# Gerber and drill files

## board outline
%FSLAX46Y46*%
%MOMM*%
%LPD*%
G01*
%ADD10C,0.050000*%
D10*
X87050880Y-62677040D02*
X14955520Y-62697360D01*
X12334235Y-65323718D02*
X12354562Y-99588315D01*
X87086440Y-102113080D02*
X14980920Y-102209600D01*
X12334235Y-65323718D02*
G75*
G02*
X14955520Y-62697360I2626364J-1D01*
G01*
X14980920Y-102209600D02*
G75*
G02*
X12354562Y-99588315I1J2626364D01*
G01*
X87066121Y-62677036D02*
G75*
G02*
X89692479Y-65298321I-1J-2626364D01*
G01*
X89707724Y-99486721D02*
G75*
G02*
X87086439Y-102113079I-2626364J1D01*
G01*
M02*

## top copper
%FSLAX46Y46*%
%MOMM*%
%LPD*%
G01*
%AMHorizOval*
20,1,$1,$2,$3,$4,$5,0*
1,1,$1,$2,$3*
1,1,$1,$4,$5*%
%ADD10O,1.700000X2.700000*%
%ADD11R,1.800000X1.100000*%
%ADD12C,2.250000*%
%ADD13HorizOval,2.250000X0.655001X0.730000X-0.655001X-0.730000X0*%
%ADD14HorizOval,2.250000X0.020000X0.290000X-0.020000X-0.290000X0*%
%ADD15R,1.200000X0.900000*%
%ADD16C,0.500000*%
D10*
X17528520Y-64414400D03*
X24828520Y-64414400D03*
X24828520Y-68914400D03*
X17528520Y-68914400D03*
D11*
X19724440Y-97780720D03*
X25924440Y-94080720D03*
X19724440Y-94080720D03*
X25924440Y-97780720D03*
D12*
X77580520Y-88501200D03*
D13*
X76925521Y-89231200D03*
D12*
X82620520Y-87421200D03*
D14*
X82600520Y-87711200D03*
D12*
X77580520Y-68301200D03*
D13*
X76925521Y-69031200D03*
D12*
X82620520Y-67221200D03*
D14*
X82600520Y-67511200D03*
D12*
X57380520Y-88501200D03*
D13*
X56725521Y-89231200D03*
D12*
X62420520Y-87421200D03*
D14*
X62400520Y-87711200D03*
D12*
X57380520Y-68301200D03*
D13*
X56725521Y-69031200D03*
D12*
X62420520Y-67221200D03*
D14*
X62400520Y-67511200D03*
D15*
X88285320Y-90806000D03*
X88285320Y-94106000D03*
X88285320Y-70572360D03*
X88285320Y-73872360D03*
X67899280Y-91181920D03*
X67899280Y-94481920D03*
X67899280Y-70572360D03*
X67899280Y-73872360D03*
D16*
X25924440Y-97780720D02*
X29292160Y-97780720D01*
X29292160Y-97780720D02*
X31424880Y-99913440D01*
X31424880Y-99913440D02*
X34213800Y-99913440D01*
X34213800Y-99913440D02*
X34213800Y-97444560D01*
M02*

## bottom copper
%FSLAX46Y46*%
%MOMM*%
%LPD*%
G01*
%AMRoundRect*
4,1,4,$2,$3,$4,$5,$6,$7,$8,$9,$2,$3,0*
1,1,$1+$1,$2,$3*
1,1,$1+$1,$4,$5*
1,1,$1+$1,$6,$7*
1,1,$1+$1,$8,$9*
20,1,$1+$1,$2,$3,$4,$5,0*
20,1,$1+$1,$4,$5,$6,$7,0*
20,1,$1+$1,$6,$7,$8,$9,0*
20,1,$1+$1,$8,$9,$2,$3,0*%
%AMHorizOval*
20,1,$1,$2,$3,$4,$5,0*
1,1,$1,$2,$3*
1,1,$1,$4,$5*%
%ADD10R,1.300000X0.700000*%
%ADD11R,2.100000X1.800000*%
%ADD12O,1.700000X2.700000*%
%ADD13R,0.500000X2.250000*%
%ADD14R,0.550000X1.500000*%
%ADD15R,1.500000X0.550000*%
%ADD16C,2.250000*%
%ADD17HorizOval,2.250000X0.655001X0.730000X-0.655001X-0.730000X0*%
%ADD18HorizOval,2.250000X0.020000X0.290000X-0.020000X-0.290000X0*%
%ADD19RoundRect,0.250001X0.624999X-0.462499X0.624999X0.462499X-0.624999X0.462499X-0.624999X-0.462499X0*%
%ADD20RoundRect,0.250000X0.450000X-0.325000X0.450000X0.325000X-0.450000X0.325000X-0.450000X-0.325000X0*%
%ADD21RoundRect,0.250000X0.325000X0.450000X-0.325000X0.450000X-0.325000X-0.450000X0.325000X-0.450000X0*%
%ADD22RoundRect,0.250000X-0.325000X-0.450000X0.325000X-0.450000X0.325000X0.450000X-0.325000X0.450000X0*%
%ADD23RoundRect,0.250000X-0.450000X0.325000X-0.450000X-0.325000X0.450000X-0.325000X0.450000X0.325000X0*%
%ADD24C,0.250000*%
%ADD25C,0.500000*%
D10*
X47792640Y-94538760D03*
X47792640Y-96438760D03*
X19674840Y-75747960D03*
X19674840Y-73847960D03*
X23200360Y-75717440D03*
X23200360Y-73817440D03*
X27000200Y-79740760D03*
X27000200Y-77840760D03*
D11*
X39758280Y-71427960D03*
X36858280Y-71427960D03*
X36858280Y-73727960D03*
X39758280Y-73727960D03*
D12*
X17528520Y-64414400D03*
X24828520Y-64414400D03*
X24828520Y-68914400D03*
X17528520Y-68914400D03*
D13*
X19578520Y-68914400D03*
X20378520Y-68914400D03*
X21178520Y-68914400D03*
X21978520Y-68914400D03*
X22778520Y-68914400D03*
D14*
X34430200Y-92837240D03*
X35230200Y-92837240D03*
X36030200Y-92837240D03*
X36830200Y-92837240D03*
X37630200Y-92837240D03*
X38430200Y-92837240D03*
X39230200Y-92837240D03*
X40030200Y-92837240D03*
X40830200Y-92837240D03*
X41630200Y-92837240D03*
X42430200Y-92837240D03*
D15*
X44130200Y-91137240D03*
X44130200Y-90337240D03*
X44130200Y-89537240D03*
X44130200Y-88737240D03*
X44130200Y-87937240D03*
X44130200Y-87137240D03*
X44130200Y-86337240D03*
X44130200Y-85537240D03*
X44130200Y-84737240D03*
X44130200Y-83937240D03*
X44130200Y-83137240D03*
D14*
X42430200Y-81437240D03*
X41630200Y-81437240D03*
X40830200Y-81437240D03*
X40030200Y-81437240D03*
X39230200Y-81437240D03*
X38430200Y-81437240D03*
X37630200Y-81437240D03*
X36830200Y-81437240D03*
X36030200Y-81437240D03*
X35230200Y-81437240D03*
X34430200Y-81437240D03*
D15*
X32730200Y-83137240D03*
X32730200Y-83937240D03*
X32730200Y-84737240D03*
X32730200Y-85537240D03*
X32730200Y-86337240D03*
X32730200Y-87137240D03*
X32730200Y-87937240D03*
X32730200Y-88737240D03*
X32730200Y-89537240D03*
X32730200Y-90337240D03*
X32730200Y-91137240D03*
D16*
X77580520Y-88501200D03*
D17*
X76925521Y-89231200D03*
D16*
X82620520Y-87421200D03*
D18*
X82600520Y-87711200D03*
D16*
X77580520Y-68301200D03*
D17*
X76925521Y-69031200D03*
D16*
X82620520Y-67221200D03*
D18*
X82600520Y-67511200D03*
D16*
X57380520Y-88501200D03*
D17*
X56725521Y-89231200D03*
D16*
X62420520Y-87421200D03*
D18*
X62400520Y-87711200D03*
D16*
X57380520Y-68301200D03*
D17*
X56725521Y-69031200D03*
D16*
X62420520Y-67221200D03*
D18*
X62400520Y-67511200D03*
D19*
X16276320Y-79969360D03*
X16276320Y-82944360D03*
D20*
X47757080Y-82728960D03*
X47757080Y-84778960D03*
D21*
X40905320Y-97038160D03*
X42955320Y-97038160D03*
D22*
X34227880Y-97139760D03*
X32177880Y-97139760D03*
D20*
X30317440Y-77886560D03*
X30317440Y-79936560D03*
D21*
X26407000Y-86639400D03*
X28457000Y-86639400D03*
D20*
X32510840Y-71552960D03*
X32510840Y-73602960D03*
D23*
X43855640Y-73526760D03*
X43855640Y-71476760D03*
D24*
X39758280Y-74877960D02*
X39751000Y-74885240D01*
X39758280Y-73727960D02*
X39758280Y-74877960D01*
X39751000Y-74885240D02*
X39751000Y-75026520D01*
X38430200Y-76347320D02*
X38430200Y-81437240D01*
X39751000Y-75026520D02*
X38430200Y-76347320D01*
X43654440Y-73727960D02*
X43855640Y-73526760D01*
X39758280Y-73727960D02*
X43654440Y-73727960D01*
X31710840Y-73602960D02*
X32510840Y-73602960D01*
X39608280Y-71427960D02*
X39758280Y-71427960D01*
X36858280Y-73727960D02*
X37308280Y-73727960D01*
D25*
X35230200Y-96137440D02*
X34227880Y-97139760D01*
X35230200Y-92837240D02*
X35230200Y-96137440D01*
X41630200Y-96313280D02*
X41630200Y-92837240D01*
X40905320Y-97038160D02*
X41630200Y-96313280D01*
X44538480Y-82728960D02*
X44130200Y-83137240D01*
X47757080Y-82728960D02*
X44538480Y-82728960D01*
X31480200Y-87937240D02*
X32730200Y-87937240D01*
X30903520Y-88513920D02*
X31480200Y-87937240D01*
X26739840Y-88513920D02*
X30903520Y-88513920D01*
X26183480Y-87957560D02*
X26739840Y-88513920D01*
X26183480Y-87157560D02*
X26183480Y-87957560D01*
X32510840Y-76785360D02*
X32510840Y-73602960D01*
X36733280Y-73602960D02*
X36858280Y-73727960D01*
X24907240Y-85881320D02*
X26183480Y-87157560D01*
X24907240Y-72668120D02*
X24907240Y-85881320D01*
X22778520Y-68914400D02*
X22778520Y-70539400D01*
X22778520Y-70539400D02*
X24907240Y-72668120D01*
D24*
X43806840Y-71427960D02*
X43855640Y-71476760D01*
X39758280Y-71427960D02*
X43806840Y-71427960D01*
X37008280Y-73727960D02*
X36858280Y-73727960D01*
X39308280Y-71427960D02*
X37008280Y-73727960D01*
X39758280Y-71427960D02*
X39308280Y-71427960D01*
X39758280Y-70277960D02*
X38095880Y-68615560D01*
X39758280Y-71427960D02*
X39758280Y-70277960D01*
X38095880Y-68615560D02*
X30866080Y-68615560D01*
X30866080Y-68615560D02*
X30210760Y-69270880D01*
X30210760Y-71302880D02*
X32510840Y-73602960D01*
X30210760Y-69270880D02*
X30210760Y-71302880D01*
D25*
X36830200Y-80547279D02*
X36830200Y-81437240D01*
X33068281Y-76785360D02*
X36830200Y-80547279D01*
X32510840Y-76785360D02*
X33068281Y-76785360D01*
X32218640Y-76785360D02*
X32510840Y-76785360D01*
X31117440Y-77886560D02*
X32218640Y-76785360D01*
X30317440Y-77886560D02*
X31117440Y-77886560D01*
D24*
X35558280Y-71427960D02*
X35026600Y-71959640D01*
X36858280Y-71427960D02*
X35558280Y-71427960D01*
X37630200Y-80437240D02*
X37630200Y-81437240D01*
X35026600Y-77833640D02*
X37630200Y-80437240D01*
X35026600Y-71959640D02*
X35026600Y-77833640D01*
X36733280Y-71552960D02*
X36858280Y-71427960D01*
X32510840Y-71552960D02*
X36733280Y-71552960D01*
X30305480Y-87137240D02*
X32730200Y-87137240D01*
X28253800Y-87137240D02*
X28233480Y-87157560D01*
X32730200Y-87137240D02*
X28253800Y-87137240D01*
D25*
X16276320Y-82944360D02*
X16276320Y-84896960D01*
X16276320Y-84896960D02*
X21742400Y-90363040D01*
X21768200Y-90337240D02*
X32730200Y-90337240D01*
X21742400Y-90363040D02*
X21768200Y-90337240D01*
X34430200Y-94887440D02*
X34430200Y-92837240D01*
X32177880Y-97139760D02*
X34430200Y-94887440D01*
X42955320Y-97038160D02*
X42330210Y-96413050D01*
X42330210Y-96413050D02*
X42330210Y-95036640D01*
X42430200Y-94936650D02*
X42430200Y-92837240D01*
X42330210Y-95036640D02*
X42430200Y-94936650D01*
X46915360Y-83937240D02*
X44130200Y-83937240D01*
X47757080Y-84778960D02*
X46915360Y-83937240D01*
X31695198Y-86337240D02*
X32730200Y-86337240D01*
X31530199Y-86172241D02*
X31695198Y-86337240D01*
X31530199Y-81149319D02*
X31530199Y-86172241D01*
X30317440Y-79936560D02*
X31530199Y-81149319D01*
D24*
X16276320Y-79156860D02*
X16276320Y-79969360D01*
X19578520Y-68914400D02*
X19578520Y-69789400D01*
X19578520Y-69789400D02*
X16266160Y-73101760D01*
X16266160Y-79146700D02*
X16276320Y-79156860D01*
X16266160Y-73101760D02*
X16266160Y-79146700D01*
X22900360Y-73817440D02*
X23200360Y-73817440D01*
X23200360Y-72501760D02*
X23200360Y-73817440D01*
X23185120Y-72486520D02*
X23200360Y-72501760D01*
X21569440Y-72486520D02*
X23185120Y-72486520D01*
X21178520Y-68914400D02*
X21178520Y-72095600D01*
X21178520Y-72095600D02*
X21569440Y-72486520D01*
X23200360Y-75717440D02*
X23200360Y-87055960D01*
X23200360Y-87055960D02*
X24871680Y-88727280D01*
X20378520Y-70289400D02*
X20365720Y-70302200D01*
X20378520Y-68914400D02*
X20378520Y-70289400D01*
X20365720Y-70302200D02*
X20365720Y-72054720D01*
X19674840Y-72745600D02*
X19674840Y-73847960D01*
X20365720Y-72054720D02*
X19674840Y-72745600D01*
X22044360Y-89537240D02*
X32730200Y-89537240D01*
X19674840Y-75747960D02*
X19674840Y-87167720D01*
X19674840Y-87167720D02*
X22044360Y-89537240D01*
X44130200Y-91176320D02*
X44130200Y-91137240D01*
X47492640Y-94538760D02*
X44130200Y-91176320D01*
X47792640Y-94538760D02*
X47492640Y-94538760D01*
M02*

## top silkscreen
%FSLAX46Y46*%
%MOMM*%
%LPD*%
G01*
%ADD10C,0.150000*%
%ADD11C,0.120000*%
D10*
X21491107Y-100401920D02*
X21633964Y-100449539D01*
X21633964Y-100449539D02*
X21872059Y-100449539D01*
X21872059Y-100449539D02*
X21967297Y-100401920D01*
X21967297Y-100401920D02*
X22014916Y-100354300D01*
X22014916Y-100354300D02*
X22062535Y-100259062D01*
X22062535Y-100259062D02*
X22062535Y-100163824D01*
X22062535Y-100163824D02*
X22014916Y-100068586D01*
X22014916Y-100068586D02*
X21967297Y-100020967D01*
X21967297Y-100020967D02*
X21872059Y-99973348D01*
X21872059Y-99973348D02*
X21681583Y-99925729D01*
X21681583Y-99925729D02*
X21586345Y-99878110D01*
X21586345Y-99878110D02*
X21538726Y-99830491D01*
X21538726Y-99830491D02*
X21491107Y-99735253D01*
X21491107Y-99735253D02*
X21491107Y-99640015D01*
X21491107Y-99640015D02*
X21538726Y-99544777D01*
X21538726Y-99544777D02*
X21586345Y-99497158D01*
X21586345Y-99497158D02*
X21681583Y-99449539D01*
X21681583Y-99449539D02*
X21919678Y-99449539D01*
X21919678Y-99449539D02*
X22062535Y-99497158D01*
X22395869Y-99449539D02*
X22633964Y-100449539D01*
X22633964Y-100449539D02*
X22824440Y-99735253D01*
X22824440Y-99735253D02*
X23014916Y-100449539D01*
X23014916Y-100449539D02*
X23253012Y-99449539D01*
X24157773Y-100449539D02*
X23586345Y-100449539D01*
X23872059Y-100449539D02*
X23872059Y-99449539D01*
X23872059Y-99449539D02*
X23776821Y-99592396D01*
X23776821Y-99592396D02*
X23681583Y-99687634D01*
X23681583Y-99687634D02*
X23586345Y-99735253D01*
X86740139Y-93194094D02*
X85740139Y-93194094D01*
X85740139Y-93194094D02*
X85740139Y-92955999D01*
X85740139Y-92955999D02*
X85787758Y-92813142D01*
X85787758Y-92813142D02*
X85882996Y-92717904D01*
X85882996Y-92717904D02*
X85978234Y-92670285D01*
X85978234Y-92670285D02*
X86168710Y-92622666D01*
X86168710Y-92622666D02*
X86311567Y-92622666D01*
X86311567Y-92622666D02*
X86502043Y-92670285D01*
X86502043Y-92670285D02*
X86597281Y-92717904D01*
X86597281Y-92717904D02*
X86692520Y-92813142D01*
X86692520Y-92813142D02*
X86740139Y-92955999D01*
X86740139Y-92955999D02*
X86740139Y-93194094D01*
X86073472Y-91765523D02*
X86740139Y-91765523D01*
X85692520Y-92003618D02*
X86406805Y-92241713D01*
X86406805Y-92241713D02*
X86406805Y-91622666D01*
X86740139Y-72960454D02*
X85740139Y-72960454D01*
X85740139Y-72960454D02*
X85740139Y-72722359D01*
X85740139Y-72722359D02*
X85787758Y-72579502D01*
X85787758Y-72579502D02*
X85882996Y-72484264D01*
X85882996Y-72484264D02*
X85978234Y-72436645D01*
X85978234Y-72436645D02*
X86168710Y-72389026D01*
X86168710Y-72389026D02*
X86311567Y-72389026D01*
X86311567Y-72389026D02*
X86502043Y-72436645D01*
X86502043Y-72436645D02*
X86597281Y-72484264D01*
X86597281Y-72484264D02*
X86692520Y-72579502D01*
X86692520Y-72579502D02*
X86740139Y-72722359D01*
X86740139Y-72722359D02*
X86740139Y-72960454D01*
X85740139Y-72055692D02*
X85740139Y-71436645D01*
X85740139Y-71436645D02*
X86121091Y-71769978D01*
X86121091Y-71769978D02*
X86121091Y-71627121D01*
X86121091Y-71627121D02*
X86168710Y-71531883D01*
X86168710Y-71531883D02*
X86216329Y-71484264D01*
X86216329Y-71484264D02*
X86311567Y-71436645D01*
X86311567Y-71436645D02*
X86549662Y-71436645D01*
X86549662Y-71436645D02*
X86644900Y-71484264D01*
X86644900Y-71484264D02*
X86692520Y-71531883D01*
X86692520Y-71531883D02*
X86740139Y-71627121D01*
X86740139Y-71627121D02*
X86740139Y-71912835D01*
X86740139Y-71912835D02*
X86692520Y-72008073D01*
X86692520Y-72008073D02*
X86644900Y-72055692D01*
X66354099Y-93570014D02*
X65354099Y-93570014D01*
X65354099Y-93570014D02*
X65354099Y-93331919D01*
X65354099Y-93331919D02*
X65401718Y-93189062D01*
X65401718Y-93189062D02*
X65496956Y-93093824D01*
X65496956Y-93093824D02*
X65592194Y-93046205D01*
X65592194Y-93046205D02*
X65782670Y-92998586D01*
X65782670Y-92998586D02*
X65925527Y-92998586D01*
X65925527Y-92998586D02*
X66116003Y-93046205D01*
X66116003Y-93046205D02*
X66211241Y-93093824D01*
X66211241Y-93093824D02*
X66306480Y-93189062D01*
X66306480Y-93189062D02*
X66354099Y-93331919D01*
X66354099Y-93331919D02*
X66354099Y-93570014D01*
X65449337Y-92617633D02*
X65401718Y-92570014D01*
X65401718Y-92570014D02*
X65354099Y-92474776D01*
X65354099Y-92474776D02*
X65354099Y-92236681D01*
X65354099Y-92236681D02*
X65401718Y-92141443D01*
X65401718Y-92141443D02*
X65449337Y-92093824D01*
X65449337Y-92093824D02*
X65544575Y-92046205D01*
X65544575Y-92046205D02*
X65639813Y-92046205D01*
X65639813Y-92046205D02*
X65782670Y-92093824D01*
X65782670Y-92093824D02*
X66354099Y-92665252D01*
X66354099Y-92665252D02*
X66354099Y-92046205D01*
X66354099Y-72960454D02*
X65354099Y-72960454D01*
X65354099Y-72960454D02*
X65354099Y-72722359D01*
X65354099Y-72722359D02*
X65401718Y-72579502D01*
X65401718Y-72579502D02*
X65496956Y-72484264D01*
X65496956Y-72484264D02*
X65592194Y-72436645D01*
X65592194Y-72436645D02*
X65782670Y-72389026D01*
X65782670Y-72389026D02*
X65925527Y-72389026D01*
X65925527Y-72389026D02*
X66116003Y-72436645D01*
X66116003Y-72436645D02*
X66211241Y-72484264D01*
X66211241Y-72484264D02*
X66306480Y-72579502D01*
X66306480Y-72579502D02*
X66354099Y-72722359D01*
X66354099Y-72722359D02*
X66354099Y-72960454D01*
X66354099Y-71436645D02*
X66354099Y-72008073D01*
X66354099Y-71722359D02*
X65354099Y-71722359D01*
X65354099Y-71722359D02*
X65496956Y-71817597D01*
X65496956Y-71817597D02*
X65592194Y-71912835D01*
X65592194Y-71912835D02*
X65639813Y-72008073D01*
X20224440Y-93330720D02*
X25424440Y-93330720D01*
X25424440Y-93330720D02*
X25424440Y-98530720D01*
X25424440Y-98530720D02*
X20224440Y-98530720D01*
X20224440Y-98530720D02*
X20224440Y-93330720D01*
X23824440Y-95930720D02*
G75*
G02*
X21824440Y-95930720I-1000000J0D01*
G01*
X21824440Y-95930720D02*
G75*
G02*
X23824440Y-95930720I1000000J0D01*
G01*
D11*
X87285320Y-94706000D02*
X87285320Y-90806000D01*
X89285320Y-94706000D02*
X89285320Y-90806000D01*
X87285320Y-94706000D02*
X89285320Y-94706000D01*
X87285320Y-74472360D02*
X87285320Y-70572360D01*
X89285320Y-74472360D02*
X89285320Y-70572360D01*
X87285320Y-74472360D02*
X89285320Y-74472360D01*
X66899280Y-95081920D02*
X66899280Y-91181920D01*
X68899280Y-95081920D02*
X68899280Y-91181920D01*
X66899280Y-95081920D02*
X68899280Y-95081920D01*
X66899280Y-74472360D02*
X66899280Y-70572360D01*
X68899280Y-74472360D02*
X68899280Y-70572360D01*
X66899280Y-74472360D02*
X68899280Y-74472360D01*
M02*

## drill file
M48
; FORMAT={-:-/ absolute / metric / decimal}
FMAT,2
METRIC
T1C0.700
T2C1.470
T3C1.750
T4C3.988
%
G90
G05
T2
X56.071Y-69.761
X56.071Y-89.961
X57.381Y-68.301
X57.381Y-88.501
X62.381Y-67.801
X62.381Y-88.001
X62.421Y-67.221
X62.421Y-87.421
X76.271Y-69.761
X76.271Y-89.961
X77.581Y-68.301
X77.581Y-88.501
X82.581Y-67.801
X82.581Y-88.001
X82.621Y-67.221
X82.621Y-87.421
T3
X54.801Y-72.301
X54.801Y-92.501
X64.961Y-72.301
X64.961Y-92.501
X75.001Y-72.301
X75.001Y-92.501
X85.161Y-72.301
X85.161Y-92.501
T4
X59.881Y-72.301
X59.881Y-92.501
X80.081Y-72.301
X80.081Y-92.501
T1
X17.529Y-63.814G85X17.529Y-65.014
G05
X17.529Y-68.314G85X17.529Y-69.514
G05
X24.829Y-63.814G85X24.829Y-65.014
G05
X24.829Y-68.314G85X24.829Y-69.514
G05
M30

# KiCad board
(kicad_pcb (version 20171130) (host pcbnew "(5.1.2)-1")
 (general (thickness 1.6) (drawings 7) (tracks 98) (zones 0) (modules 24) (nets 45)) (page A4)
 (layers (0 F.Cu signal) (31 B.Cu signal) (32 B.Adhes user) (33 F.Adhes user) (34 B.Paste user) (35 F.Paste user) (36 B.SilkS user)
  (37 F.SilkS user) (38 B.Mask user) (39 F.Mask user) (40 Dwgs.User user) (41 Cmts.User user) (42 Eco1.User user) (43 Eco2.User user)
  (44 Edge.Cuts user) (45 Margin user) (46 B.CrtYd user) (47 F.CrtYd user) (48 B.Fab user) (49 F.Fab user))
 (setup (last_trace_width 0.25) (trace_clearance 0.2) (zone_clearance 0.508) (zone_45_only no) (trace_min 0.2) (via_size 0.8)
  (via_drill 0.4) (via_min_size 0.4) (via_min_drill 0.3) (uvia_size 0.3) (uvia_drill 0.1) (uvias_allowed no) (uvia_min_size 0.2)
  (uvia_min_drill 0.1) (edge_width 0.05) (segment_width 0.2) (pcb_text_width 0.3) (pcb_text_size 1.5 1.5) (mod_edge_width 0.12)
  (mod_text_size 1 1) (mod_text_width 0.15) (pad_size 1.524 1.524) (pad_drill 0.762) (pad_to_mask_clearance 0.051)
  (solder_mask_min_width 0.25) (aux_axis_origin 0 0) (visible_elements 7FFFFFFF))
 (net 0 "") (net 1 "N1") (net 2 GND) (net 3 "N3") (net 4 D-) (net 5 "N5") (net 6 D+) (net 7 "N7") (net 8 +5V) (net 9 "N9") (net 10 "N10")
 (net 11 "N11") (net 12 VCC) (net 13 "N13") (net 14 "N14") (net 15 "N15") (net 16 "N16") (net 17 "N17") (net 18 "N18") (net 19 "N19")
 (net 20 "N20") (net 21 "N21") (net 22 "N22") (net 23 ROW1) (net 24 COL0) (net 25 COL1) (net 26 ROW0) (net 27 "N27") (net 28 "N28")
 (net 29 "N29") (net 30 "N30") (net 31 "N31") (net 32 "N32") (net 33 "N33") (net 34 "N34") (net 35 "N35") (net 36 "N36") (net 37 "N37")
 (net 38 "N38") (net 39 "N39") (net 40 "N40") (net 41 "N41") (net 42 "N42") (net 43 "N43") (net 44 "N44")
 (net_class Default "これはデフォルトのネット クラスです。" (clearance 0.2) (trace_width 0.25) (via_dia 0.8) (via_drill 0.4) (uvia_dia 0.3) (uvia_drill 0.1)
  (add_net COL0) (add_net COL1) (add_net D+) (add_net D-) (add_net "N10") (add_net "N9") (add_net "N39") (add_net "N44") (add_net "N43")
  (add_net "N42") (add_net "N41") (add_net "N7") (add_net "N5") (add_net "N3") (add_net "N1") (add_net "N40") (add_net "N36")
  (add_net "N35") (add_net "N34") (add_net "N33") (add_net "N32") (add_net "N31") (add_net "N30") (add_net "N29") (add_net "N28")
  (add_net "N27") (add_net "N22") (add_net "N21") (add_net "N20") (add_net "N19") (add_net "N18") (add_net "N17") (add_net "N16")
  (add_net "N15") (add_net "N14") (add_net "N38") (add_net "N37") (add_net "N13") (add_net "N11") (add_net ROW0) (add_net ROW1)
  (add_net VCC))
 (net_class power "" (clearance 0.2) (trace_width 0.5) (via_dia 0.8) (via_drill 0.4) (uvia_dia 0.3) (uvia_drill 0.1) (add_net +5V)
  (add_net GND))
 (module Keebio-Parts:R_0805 (layer B.Cu) (at 47.79264 95.48876 90)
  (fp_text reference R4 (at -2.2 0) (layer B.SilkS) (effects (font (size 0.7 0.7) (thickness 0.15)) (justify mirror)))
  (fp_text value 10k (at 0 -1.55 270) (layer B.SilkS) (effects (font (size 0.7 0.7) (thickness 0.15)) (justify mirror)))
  (pad 2 smd rect (at 0.95 0 90) (size 0.7 1.3) (layers B.Cu B.Paste B.Mask) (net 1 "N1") (clearance 0.1))
  (pad 1 smd rect (at -0.95 0 90) (size 0.7 1.3) (layers B.Cu B.Paste B.Mask) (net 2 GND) (clearance 0.1)))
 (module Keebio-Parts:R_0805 (layer B.Cu) (at 19.67484 74.79796 90)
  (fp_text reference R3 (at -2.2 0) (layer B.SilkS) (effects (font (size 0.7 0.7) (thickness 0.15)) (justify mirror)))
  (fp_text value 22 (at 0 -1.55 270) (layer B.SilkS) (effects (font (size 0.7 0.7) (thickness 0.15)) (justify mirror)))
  (pad 1 smd rect (at -0.95 0 90) (size 0.7 1.3) (layers B.Cu B.Paste B.Mask) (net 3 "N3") (clearance 0.1))
  (pad 2 smd rect (at 0.95 0 90) (size 0.7 1.3) (layers B.Cu B.Paste B.Mask) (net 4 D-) (clearance 0.1)))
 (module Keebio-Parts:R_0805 (layer B.Cu) (at 23.20036 74.76744 90)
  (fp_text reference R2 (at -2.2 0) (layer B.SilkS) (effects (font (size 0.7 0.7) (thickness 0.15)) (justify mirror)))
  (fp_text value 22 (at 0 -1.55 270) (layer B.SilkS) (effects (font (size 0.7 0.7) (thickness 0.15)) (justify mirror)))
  (pad 1 smd rect (at -0.95 0 90) (size 0.7 1.3) (layers B.Cu B.Paste B.Mask) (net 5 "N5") (clearance 0.1))
  (pad 2 smd rect (at 0.95 0 90) (size 0.7 1.3) (layers B.Cu B.Paste B.Mask) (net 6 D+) (clearance 0.1)))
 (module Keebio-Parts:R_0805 (layer B.Cu) (at 27.0002 78.79076 90)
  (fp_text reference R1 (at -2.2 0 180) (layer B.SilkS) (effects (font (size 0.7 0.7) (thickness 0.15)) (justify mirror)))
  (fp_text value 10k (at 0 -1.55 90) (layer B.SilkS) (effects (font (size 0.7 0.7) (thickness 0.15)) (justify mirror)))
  (pad 1 smd rect (at -0.95 0 90) (size 0.7 1.3) (layers B.Cu B.Paste B.Mask) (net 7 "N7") (clearance 0.1))
  (pad 2 smd rect (at 0.95 0 90) (size 0.7 1.3) (layers B.Cu B.Paste B.Mask) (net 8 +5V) (clearance 0.1)))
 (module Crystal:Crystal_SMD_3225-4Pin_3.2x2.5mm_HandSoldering (layer B.Cu) (at 38.30828 72.57796 180)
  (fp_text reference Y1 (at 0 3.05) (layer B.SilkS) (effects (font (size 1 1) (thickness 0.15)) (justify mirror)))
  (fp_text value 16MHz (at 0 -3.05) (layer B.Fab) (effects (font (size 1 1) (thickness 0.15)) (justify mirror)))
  (pad 4 smd rect (at -1.45 1.15 180) (size 2.1 1.8) (layers B.Cu B.Paste B.Mask) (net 2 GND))
  (pad 3 smd rect (at 1.45 1.15 180) (size 2.1 1.8) (layers B.Cu B.Paste B.Mask) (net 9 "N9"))
  (pad 2 smd rect (at 1.45 -1.15 180) (size 2.1 1.8) (layers B.Cu B.Paste B.Mask) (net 2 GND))
  (pad 1 smd rect (at -1.45 -1.15 180) (size 2.1 1.8) (layers B.Cu B.Paste B.Mask) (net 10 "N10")))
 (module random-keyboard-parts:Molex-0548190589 (layer B.Cu) (at 21.17852 64.4144 270)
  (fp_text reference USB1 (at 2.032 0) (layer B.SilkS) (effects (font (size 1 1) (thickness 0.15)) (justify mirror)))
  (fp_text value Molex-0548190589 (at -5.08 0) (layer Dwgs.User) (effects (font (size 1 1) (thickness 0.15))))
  (pad 6 thru_hole oval (at 0 3.65 270) (size 2.7 1.7) (drill oval 1.9 0.7) (layers *.Cu *.Mask) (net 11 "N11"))
  (pad 6 thru_hole oval (at 0 -3.65 270) (size 2.7 1.7) (drill oval 1.9 0.7) (layers *.Cu *.Mask) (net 11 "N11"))
  (pad 6 thru_hole oval (at 4.5 -3.65 270) (size 2.7 1.7) (drill oval 1.9 0.7) (layers *.Cu *.Mask) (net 11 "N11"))
  (pad 6 thru_hole oval (at 4.5 3.65 270) (size 2.7 1.7) (drill oval 1.9 0.7) (layers *.Cu *.Mask) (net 11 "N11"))
  (pad 5 smd rect (at 4.5 1.6 270) (size 2.25 0.5) (layers B.Cu B.Paste B.Mask) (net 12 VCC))
  (pad 4 smd rect (at 4.5 0.8 270) (size 2.25 0.5) (layers B.Cu B.Paste B.Mask) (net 4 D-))
  (pad 3 smd rect (at 4.5 0 270) (size 2.25 0.5) (layers B.Cu B.Paste B.Mask) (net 6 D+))
  (pad 2 smd rect (at 4.5 -0.8 270) (size 2.25 0.5) (layers B.Cu B.Paste B.Mask) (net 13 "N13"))
  (pad 1 smd rect (at 4.5 -1.6 270) (size 2.25 0.5) (layers B.Cu B.Paste B.Mask) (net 2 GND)))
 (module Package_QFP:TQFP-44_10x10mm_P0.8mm (layer B.Cu) (at 38.4302 87.13724)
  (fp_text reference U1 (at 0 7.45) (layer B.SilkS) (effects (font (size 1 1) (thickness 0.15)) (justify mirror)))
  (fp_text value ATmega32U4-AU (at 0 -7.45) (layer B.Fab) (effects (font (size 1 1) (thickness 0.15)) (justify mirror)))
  (pad 44 smd rect (at -4 5.7 270) (size 1.5 0.55) (layers B.Cu B.Paste B.Mask) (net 8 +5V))
  (pad 43 smd rect (at -3.2 5.7 270) (size 1.5 0.55) (layers B.Cu B.Paste B.Mask) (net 2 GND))
  (pad 42 smd rect (at -2.4 5.7 270) (size 1.5 0.55) (layers B.Cu B.Paste B.Mask) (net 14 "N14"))
  (pad 41 smd rect (at -1.6 5.7 270) (size 1.5 0.55) (layers B.Cu B.Paste B.Mask) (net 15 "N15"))
  (pad 40 smd rect (at -0.8 5.7 270) (size 1.5 0.55) (layers B.Cu B.Paste B.Mask) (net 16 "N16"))
  (pad 39 smd rect (at 0 5.7 270) (size 1.5 0.55) (layers B.Cu B.Paste B.Mask) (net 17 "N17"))
  (pad 38 smd rect (at 0.8 5.7 270) (size 1.5 0.55) (layers B.Cu B.Paste B.Mask) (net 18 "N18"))
  (pad 37 smd rect (at 1.6 5.7 270) (size 1.5 0.55) (layers B.Cu B.Paste B.Mask) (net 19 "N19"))
  (pad 36 smd rect (at 2.4 5.7 270) (size 1.5 0.55) (layers B.Cu B.Paste B.Mask) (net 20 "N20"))
  (pad 35 smd rect (at 3.2 5.7 270) (size 1.5 0.55) (layers B.Cu B.Paste B.Mask) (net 2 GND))
  (pad 34 smd rect (at 4 5.7 270) (size 1.5 0.55) (layers B.Cu B.Paste B.Mask) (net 8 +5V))
  (pad 33 smd rect (at 5.7 4) (size 1.5 0.55) (layers B.Cu B.Paste B.Mask) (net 1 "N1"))
  (pad 32 smd rect (at 5.7 3.2) (size 1.5 0.55) (layers B.Cu B.Paste B.Mask) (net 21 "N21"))
  (pad 31 smd rect (at 5.7 2.4) (size 1.5 0.55) (layers B.Cu B.Paste B.Mask) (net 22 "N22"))
  (pad 30 smd rect (at 5.7 1.6) (size 1.5 0.55) (layers B.Cu B.Paste B.Mask) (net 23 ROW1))
  (pad 29 smd rect (at 5.7 0.8) (size 1.5 0.55) (layers B.Cu B.Paste B.Mask) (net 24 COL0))
  (pad 28 smd rect (at 5.7 0) (size 1.5 0.55) (layers B.Cu B.Paste B.Mask) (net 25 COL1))
  (pad 27 smd rect (at 5.7 -0.8) (size 1.5 0.55) (layers B.Cu B.Paste B.Mask) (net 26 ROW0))
  (pad 26 smd rect (at 5.7 -1.6) (size 1.5 0.55) (layers B.Cu B.Paste B.Mask) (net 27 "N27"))
  (pad 25 smd rect (at 5.7 -2.4) (size 1.5 0.55) (layers B.Cu B.Paste B.Mask) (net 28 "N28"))
  (pad 24 smd rect (at 5.7 -3.2) (size 1.5 0.55) (layers B.Cu B.Paste B.Mask) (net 8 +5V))
  (pad 23 smd rect (at 5.7 -4) (size 1.5 0.55) (layers B.Cu B.Paste B.Mask) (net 2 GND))
  (pad 22 smd rect (at 4 -5.7 270) (size 1.5 0.55) (layers B.Cu B.Paste B.Mask) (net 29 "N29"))
  (pad 21 smd rect (at 3.2 -5.7 270) (size 1.5 0.55) (layers B.Cu B.Paste B.Mask) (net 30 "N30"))
  (pad 20 smd rect (at 2.4 -5.7 270) (size 1.5 0.55) (layers B.Cu B.Paste B.Mask) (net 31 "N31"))
  (pad 19 smd rect (at 1.6 -5.7 270) (size 1.5 0.55) (layers B.Cu B.Paste B.Mask) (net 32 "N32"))
  (pad 18 smd rect (at 0.8 -5.7 270) (size 1.5 0.55) (layers B.Cu B.Paste B.Mask) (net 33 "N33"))
  (pad 17 smd rect (at 0 -5.7 270) (size 1.5 0.55) (layers B.Cu B.Paste B.Mask) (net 10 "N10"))
  (pad 16 smd rect (at -0.8 -5.7 270) (size 1.5 0.55) (layers B.Cu B.Paste B.Mask) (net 9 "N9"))
  (pad 15 smd rect (at -1.6 -5.7 270) (size 1.5 0.55) (layers B.Cu B.Paste B.Mask) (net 2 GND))
  (pad 14 smd rect (at -2.4 -5.7 270) (size 1.5 0.55) (layers B.Cu B.Paste B.Mask) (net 8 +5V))
  (pad 13 smd rect (at -3.2 -5.7 270) (size 1.5 0.55) (layers B.Cu B.Paste B.Mask) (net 7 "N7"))
  (pad 12 smd rect (at -4 -5.7 270) (size 1.5 0.55) (layers B.Cu B.Paste B.Mask) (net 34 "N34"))
  (pad 11 smd rect (at -5.7 -4) (size 1.5 0.55) (layers B.Cu B.Paste B.Mask) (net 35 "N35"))
  (pad 10 smd rect (at -5.7 -3.2) (size 1.5 0.55) (layers B.Cu B.Paste B.Mask) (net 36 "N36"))
  (pad 9 smd rect (at -5.7 -2.4) (size 1.5 0.55) (layers B.Cu B.Paste B.Mask) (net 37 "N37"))
  (pad 8 smd rect (at -5.7 -1.6) (size 1.5 0.55) (layers B.Cu B.Paste B.Mask) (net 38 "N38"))
  (pad 7 smd rect (at -5.7 -0.8) (size 1.5 0.55) (layers B.Cu B.Paste B.Mask) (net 8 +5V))
  (pad 6 smd rect (at -5.7 0) (size 1.5 0.55) (layers B.Cu B.Paste B.Mask) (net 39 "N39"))
  (pad 5 smd rect (at -5.7 0.8) (size 1.5 0.55) (layers B.Cu B.Paste B.Mask) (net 2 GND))
  (pad 4 smd rect (at -5.7 1.6) (size 1.5 0.55) (layers B.Cu B.Paste B.Mask) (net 5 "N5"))
  (pad 3 smd rect (at -5.7 2.4) (size 1.5 0.55) (layers B.Cu B.Paste B.Mask) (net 3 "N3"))
  (pad 2 smd rect (at -5.7 3.2) (size 1.5 0.55) (layers B.Cu B.Paste B.Mask) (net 8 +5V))
  (pad 1 smd rect (at -5.7 4) (size 1.5 0.55) (layers B.Cu B.Paste B.Mask) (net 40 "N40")))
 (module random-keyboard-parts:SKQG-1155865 (layer F.Cu) (at 22.82444 95.93072)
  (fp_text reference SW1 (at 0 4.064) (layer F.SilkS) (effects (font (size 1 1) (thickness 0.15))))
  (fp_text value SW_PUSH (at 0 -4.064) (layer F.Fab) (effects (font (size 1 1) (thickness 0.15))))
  (fp_line (start -2.6 -2.6) (end 2.6 -2.6) (layer F.SilkS) (width 0.15))
  (fp_line (start 2.6 -2.6) (end 2.6 2.6) (layer F.SilkS) (width 0.15))
  (fp_line (start 2.6 2.6) (end -2.6 2.6) (layer F.SilkS) (width 0.15))
  (fp_line (start -2.6 2.6) (end -2.6 -2.6) (layer F.SilkS) (width 0.15))
  (fp_circle (center 0 0) (end 1 0) (layer F.SilkS) (width 0.15))
  (pad 4 smd rect (at -3.1 1.85) (size 1.8 1.1) (layers F.Cu F.Paste F.Mask))
  (pad 3 smd rect (at 3.1 -1.85) (size 1.8 1.1) (layers F.Cu F.Paste F.Mask))
  (pad 2 smd rect (at -3.1 -1.85) (size 1.8 1.1) (layers F.Cu F.Paste F.Mask) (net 7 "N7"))
  (pad 1 smd rect (at 3.1 1.85) (size 1.8 1.1) (layers F.Cu F.Paste F.Mask) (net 2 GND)))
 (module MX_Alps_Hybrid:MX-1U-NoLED (layer F.Cu) (at 80.08052 92.5012)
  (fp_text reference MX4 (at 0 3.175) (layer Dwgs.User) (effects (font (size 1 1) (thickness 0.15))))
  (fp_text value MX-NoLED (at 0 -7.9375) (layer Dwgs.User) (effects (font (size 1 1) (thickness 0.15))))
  (pad "" np_thru_hole circle (at 5.08 0 48.0996) (size 1.75 1.75) (drill 1.75) (layers *.Cu *.Mask))
  (pad "" np_thru_hole circle (at -5.08 0 48.0996) (size 1.75 1.75) (drill 1.75) (layers *.Cu *.Mask))
  (pad 1 thru_hole circle (at -2.5 -4) (size 2.25 2.25) (drill 1.47) (layers *.Cu B.Mask) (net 25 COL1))
  (pad "" np_thru_hole circle (at 0 0) (size 3.9878 3.9878) (drill 3.9878) (layers *.Cu *.Mask))
  (pad 1 thru_hole oval (at -3.81 -2.54 48.0996) (size 4.211556 2.25) (drill 1.47 (offset 0.980778 0)) (layers *.Cu B.Mask) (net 25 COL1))
  (pad 2 thru_hole circle (at 2.54 -5.08) (size 2.25 2.25) (drill 1.47) (layers *.Cu B.Mask) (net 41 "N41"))
  (pad 2 thru_hole oval (at 2.5 -4.5 86.0548) (size 2.831378 2.25) (drill 1.47 (offset 0.290689 0)) (layers *.Cu B.Mask) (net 41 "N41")))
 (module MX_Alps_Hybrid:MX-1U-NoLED (layer F.Cu) (at 80.08052 72.3012)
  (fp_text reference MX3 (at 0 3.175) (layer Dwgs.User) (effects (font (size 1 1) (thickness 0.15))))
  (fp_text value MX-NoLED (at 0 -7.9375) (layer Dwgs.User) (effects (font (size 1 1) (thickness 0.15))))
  (pad "" np_thru_hole circle (at 5.08 0 48.0996) (size 1.75 1.75) (drill 1.75) (layers *.Cu *.Mask))
  (pad "" np_thru_hole circle (at -5.08 0 48.0996) (size 1.75 1.75) (drill 1.75) (layers *.Cu *.Mask))
  (pad 1 thru_hole circle (at -2.5 -4) (size 2.25 2.25) (drill 1.47) (layers *.Cu B.Mask) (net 24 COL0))
  (pad "" np_thru_hole circle (at 0 0) (size 3.9878 3.9878) (drill 3.9878) (layers *.Cu *.Mask))
  (pad 1 thru_hole oval (at -3.81 -2.54 48.0996) (size 4.211556 2.25) (drill 1.47 (offset 0.980778 0)) (layers *.Cu B.Mask) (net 24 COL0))
  (pad 2 thru_hole circle (at 2.54 -5.08) (size 2.25 2.25) (drill 1.47) (layers *.Cu B.Mask) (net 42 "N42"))
  (pad 2 thru_hole oval (at 2.5 -4.5 86.0548) (size 2.831378 2.25) (drill 1.47 (offset 0.290689 0)) (layers *.Cu B.Mask) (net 42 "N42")))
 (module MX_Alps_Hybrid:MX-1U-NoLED (layer F.Cu) (at 59.88052 92.5012)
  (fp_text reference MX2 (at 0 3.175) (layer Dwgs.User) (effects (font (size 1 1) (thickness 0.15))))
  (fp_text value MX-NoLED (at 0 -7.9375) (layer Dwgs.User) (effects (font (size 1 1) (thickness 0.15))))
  (pad "" np_thru_hole circle (at 5.08 0 48.0996) (size 1.75 1.75) (drill 1.75) (layers *.Cu *.Mask))
  (pad "" np_thru_hole circle (at -5.08 0 48.0996) (size 1.75 1.75) (drill 1.75) (layers *.Cu *.Mask))
  (pad 1 thru_hole circle (at -2.5 -4) (size 2.25 2.25) (drill 1.47) (layers *.Cu B.Mask) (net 25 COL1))
  (pad "" np_thru_hole circle (at 0 0) (size 3.9878 3.9878) (drill 3.9878) (layers *.Cu *.Mask))
  (pad 1 thru_hole oval (at -3.81 -2.54 48.0996) (size 4.211556 2.25) (drill 1.47 (offset 0.980778 0)) (layers *.Cu B.Mask) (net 25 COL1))
  (pad 2 thru_hole circle (at 2.54 -5.08) (size 2.25 2.25) (drill 1.47) (layers *.Cu B.Mask) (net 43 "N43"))
  (pad 2 thru_hole oval (at 2.5 -4.5 86.0548) (size 2.831378 2.25) (drill 1.47 (offset 0.290689 0)) (layers *.Cu B.Mask) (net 43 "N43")))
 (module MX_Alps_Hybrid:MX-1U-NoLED (layer F.Cu) (at 59.88052 72.3012)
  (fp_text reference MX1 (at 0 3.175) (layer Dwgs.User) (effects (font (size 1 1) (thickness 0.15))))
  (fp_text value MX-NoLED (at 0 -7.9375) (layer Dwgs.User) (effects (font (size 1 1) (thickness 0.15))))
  (pad "" np_thru_hole circle (at 5.08 0 48.0996) (size 1.75 1.75) (drill 1.75) (layers *.Cu *.Mask))
  (pad "" np_thru_hole circle (at -5.08 0 48.0996) (size 1.75 1.75) (drill 1.75) (layers *.Cu *.Mask))
  (pad 1 thru_hole circle (at -2.5 -4) (size 2.25 2.25) (drill 1.47) (layers *.Cu B.Mask) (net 24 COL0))
  (pad "" np_thru_hole circle (at 0 0) (size 3.9878 3.9878) (drill 3.9878) (layers *.Cu *.Mask))
  (pad 1 thru_hole oval (at -3.81 -2.54 48.0996) (size 4.211556 2.25) (drill 1.47 (offset 0.980778 0)) (layers *.Cu B.Mask) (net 24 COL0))
  (pad 2 thru_hole circle (at 2.54 -5.08) (size 2.25 2.25) (drill 1.47) (layers *.Cu B.Mask) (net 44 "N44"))
  (pad 2 thru_hole oval (at 2.5 -4.5 86.0548) (size 2.831378 2.25) (drill 1.47 (offset 0.290689 0)) (layers *.Cu B.Mask) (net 44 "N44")))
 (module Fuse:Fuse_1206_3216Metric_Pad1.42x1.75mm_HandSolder (layer B.Cu) (at 16.27632 81.45686 90)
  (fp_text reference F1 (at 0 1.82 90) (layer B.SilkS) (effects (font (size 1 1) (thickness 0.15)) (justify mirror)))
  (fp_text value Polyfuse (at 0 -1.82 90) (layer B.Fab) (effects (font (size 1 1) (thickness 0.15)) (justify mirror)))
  (pad 2 smd roundrect (at 1.4875 0 90) (size 1.425 1.75) (layers B.Cu B.Paste B.Mask) (roundrect_rratio 0.175439) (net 12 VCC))
  (pad 1 smd roundrect (at -1.4875 0 90) (size 1.425 1.75) (layers B.Cu B.Paste B.Mask) (roundrect_rratio 0.175439) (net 8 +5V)))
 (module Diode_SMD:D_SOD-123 (layer F.Cu) (at 88.28532 92.456 90)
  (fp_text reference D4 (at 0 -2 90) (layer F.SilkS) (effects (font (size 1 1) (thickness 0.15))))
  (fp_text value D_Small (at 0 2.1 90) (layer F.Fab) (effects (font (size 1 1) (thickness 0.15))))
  (fp_line (start -2.25 -1) (end 1.65 -1) (layer F.SilkS) (width 0.12))
  (fp_line (start -2.25 1) (end 1.65 1) (layer F.SilkS) (width 0.12))
  (fp_line (start -2.25 -1) (end -2.25 1) (layer F.SilkS) (width 0.12))
  (pad 2 smd rect (at 1.65 0 90) (size 0.9 1.2) (layers F.Cu F.Paste F.Mask) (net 41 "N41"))
  (pad 1 smd rect (at -1.65 0 90) (size 0.9 1.2) (layers F.Cu F.Paste F.Mask) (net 23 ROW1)))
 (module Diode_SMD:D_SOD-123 (layer F.Cu) (at 88.28532 72.22236 90)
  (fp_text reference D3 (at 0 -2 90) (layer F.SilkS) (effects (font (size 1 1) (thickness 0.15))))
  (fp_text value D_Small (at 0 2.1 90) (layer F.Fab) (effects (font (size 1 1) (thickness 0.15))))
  (fp_line (start -2.25 -1) (end 1.65 -1) (layer F.SilkS) (width 0.12))
  (fp_line (start -2.25 1) (end 1.65 1) (layer F.SilkS) (width 0.12))
  (fp_line (start -2.25 -1) (end -2.25 1) (layer F.SilkS) (width 0.12))
  (pad 2 smd rect (at 1.65 0 90) (size 0.9 1.2) (layers F.Cu F.Paste F.Mask) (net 42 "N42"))
  (pad 1 smd rect (at -1.65 0 90) (size 0.9 1.2) (layers F.Cu F.Paste F.Mask) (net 23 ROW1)))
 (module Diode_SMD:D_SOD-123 (layer F.Cu) (at 67.89928 92.83192 90)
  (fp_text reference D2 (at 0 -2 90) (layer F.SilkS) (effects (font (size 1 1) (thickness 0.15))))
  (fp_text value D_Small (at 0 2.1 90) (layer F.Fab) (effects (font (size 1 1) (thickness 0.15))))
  (fp_line (start -2.25 -1) (end 1.65 -1) (layer F.SilkS) (width 0.12))
  (fp_line (start -2.25 1) (end 1.65 1) (layer F.SilkS) (width 0.12))
  (fp_line (start -2.25 -1) (end -2.25 1) (layer F.SilkS) (width 0.12))
  (pad 2 smd rect (at 1.65 0 90) (size 0.9 1.2) (layers F.Cu F.Paste F.Mask) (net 43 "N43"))
  (pad 1 smd rect (at -1.65 0 90) (size 0.9 1.2) (layers F.Cu F.Paste F.Mask) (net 26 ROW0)))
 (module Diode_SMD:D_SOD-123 (layer F.Cu) (at 67.89928 72.22236 90)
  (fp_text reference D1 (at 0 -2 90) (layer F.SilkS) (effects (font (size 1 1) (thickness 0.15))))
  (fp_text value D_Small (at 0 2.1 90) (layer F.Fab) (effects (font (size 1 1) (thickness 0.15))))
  (fp_line (start -2.25 -1) (end 1.65 -1) (layer F.SilkS) (width 0.12))
  (fp_line (start -2.25 1) (end 1.65 1) (layer F.SilkS) (width 0.12))
  (fp_line (start -2.25 -1) (end -2.25 1) (layer F.SilkS) (width 0.12))
  (pad 2 smd rect (at 1.65 0 90) (size 0.9 1.2) (layers F.Cu F.Paste F.Mask) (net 44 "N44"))
  (pad 1 smd rect (at -1.65 0 90) (size 0.9 1.2) (layers F.Cu F.Paste F.Mask) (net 26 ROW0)))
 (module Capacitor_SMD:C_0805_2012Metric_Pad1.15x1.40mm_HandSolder (layer B.Cu) (at 47.75708 83.75396 90)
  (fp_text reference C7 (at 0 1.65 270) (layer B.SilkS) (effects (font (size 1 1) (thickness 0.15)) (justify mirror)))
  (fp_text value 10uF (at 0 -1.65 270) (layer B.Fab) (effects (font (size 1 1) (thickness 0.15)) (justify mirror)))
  (pad 2 smd roundrect (at 1.025 0 90) (size 1.15 1.4) (layers B.Cu B.Paste B.Mask) (roundrect_rratio 0.217391) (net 2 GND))
  (pad 1 smd roundrect (at -1.025 0 90) (size 1.15 1.4) (layers B.Cu B.Paste B.Mask) (roundrect_rratio 0.217391) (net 8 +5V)))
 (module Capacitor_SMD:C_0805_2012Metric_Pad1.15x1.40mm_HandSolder (layer B.Cu) (at 41.93032 97.03816 180)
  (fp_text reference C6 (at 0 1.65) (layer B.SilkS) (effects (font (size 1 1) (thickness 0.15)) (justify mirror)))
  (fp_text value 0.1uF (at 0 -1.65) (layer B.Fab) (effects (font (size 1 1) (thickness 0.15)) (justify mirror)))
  (pad 2 smd roundrect (at 1.025 0 180) (size 1.15 1.4) (layers B.Cu B.Paste B.Mask) (roundrect_rratio 0.217391) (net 2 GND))
  (pad 1 smd roundrect (at -1.025 0 180) (size 1.15 1.4) (layers B.Cu B.Paste B.Mask) (roundrect_rratio 0.217391) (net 8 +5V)))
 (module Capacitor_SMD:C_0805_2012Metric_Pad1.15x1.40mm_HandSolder (layer B.Cu) (at 33.20288 97.13976)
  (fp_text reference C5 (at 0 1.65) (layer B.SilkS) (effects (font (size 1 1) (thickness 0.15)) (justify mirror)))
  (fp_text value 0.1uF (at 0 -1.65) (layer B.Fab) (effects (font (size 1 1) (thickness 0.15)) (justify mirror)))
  (pad 2 smd roundrect (at 1.025 0) (size 1.15 1.4) (layers B.Cu B.Paste B.Mask) (roundrect_rratio 0.217391) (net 2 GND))
  (pad 1 smd roundrect (at -1.025 0) (size 1.15 1.4) (layers B.Cu B.Paste B.Mask) (roundrect_rratio 0.217391) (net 8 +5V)))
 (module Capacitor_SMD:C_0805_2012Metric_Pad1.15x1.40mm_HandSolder (layer B.Cu) (at 30.31744 78.91156 90)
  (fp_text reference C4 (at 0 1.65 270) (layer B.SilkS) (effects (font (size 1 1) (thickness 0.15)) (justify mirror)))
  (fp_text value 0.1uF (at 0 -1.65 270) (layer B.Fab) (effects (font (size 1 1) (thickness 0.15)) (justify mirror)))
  (pad 2 smd roundrect (at 1.025 0 90) (size 1.15 1.4) (layers B.Cu B.Paste B.Mask) (roundrect_rratio 0.217391) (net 2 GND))
  (pad 1 smd roundrect (at -1.025 0 90) (size 1.15 1.4) (layers B.Cu B.Paste B.Mask) (roundrect_rratio 0.217391) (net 8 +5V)))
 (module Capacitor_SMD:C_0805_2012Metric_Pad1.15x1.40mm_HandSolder (layer B.Cu) (at 27.432 86.6394 180)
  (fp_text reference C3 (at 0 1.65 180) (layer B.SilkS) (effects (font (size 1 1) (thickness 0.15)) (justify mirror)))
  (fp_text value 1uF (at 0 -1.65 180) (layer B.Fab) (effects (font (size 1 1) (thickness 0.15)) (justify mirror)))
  (pad 2 smd roundrect (at 1.025 0 180) (size 1.15 1.4) (layers B.Cu B.Paste B.Mask) (roundrect_rratio 0.217391) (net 2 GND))
  (pad 1 smd roundrect (at -1.025 0 180) (size 1.15 1.4) (layers B.Cu B.Paste B.Mask) (roundrect_rratio 0.217391) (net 39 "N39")))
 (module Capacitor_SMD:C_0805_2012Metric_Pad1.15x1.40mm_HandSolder (layer B.Cu) (at 32.51084 72.57796 90)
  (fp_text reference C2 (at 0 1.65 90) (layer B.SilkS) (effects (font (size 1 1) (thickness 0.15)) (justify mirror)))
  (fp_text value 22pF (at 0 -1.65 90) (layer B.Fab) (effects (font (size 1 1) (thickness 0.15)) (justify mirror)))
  (pad 2 smd roundrect (at 1.025 0 90) (size 1.15 1.4) (layers B.Cu B.Paste B.Mask) (roundrect_rratio 0.217391) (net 9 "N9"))
  (pad 1 smd roundrect (at -1.025 0 90) (size 1.15 1.4) (layers B.Cu B.Paste B.Mask) (roundrect_rratio 0.217391) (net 2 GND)))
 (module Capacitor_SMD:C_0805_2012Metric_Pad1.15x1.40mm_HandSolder (layer B.Cu) (at 43.85564 72.50176 270)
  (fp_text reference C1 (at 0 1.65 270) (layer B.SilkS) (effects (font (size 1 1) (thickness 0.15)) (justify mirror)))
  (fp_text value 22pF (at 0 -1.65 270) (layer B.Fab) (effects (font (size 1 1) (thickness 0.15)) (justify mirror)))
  (pad 2 smd roundrect (at 1.025 0 270) (size 1.15 1.4) (layers B.Cu B.Paste B.Mask) (roundrect_rratio 0.217391) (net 10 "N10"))
  (pad 1 smd roundrect (at -1.025 0 270) (size 1.15 1.4) (layers B.Cu B.Paste B.Mask) (roundrect_rratio 0.217391) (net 2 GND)))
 (gr_line (start 87.05088 62.67704) (end 14.95552 62.69736) (layer Edge.Cuts) (width 0.05))
 (gr_line (start 12.334235 65.323718) (end 12.354562 99.588315) (layer Edge.Cuts) (width 0.05))
 (gr_line (start 87.08644 102.11308) (end 14.98092 102.2096) (layer Edge.Cuts) (width 0.05))
 (gr_arc (start 14.960599 65.323719) (end 14.95552 62.69736) (angle -89.88917654) (layer Edge.Cuts) (width 0.05))
 (gr_arc (start 14.980921 99.583236) (end 12.354562 99.588315) (angle -89.88917654) (layer Edge.Cuts) (width 0.05))
 (gr_arc (start 87.06612 65.3034) (end 89.692479 65.298321) (angle -89.88917654) (layer Edge.Cuts) (width 0.05))
 (gr_arc (start 87.08136 99.48672) (end 87.086439 102.113079) (angle -89.88917658) (layer Edge.Cuts) (width 0.05))
 (segment (start 39.75828 74.87796) (end 39.751 74.88524) (width 0.25) (layer B.Cu) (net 10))
 (segment (start 39.75828 73.72796) (end 39.75828 74.87796) (width 0.25) (layer B.Cu) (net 10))
 (segment (start 39.751 74.88524) (end 39.751 75.02652) (width 0.25) (layer B.Cu) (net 10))
 (segment (start 38.4302 76.34732) (end 38.4302 81.43724) (width 0.25) (layer B.Cu) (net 10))
 (segment (start 39.751 75.02652) (end 38.4302 76.34732) (width 0.25) (layer B.Cu) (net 10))
 (segment (start 43.65444 73.72796) (end 43.85564 73.52676) (width 0.25) (layer B.Cu) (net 10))
 (segment (start 39.75828 73.72796) (end 43.65444 73.72796) (width 0.25) (layer B.Cu) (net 10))
 (segment (start 31.71084 73.60296) (end 32.51084 73.60296) (width 0.25) (layer B.Cu) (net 2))
 (segment (start 39.60828 71.42796) (end 39.75828 71.42796) (width 0.25) (layer B.Cu) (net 2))
 (segment (start 36.85828 73.72796) (end 37.30828 73.72796) (width 0.25) (layer B.Cu) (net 2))
 (segment (start 35.2302 96.13744) (end 34.22788 97.13976) (width 0.5) (layer B.Cu) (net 2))
 (segment (start 35.2302 92.83724) (end 35.2302 96.13744) (width 0.5) (layer B.Cu) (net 2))
 (segment (start 41.6302 96.31328) (end 41.6302 92.83724) (width 0.5) (layer B.Cu) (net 2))
 (segment (start 40.90532 97.03816) (end 41.6302 96.31328) (width 0.5) (layer B.Cu) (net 2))
 (segment (start 44.53848 82.72896) (end 44.1302 83.13724) (width 0.5) (layer B.Cu) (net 2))
 (segment (start 47.75708 82.72896) (end 44.53848 82.72896) (width 0.5) (layer B.Cu) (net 2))
 (segment (start 25.92444 97.78072) (end 29.29216 97.78072) (width 0.5) (layer F.Cu) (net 2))
 (segment (start 29.29216 97.78072) (end 31.42488 99.91344) (width 0.5) (layer F.Cu) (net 2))
 (segment (start 31.42488 99.91344) (end 34.2138 99.91344) (width 0.5) (layer F.Cu) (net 2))
 (segment (start 34.2138 99.91344) (end 34.2138 97.44456) (width 0.5) (layer F.Cu) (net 2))
 (segment (start 31.4802 87.93724) (end 32.7302 87.93724) (width 0.5) (layer B.Cu) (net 2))
 (segment (start 30.90352 88.51392) (end 31.4802 87.93724) (width 0.5) (layer B.Cu) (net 2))
 (segment (start 26.73984 88.51392) (end 30.90352 88.51392) (width 0.5) (layer B.Cu) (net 2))
 (segment (start 26.18348 87.95756) (end 26.73984 88.51392) (width 0.5) (layer B.Cu) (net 2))
 (segment (start 26.18348 87.15756) (end 26.18348 87.95756) (width 0.5) (layer B.Cu) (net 2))
 (segment (start 32.51084 76.78536) (end 32.51084 73.60296) (width 0.5) (layer B.Cu) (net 2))
 (segment (start 36.73328 73.60296) (end 36.85828 73.72796) (width 0.5) (layer B.Cu) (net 2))
 (segment (start 24.90724 85.88132) (end 26.18348 87.15756) (width 0.5) (layer B.Cu) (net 2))
 (segment (start 24.90724 72.66812) (end 24.90724 85.88132) (width 0.5) (layer B.Cu) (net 2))
 (segment (start 22.77852 68.9144) (end 22.77852 70.5394) (width 0.5) (layer B.Cu) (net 2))
 (segment (start 22.77852 70.5394) (end 24.90724 72.66812) (width 0.5) (layer B.Cu) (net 2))
 (segment (start 43.80684 71.42796) (end 43.85564 71.47676) (width 0.25) (layer B.Cu) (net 2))
 (segment (start 39.75828 71.42796) (end 43.80684 71.42796) (width 0.25) (layer B.Cu) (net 2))
 (segment (start 37.00828 73.72796) (end 36.85828 73.72796) (width 0.25) (layer B.Cu) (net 2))
 (segment (start 39.30828 71.42796) (end 37.00828 73.72796) (width 0.25) (layer B.Cu) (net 2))
 (segment (start 39.75828 71.42796) (end 39.30828 71.42796) (width 0.25) (layer B.Cu) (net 2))
 (segment (start 39.75828 70.27796) (end 38.09588 68.61556) (width 0.25) (layer B.Cu) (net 2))
 (segment (start 39.75828 71.42796) (end 39.75828 70.27796) (width 0.25) (layer B.Cu) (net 2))
 (segment (start 38.09588 68.61556) (end 30.86608 68.61556) (width 0.25) (layer B.Cu) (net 2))
 (segment (start 30.86608 68.61556) (end 30.21076 69.27088) (width 0.25) (layer B.Cu) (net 2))
 (segment (start 30.21076 71.30288) (end 32.51084 73.60296) (width 0.25) (layer B.Cu) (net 2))
 (segment (start 30.21076 69.27088) (end 30.21076 71.30288) (width 0.25) (layer B.Cu) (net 2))
 (segment (start 36.8302 80.547279) (end 36.8302 81.43724) (width 0.5) (layer B.Cu) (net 2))
 (segment (start 33.068281 76.78536) (end 36.8302 80.547279) (width 0.5) (layer B.Cu) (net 2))
 (segment (start 32.51084 76.78536) (end 33.068281 76.78536) (width 0.5) (layer B.Cu) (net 2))
 (segment (start 32.21864 76.78536) (end 32.51084 76.78536) (width 0.5) (layer B.Cu) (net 2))
 (segment (start 31.11744 77.88656) (end 32.21864 76.78536) (width 0.5) (layer B.Cu) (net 2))
 (segment (start 30.31744 77.88656) (end 31.11744 77.88656) (width 0.5) (layer B.Cu) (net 2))
 (segment (start 35.55828 71.42796) (end 35.0266 71.95964) (width 0.25) (layer B.Cu) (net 9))
 (segment (start 36.85828 71.42796) (end 35.55828 71.42796) (width 0.25) (layer B.Cu) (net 9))
 (segment (start 37.6302 80.43724) (end 37.6302 81.43724) (width 0.25) (layer B.Cu) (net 9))
 (segment (start 35.0266 77.83364) (end 37.6302 80.43724) (width 0.25) (layer B.Cu) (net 9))
 (segment (start 35.0266 71.95964) (end 35.0266 77.83364) (width 0.25) (layer B.Cu) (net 9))
 (segment (start 36.73328 71.55296) (end 36.85828 71.42796) (width 0.25) (layer B.Cu) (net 9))
 (segment (start 32.51084 71.55296) (end 36.73328 71.55296) (width 0.25) (layer B.Cu) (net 9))
 (segment (start 30.30548 87.13724) (end 32.7302 87.13724) (width 0.25) (layer B.Cu) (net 39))
 (segment (start 28.2538 87.13724) (end 28.23348 87.15756) (width 0.25) (layer B.Cu) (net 39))
 (segment (start 32.7302 87.13724) (end 28.2538 87.13724) (width 0.25) (layer B.Cu) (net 39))
 (segment (start 16.27632 82.94436) (end 16.27632 84.89696) (width 0.5) (layer B.Cu) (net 8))
 (segment (start 16.27632 84.89696) (end 21.7424 90.36304) (width 0.5) (layer B.Cu) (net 8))
 (segment (start 21.7682 90.33724) (end 32.7302 90.33724) (width 0.5) (layer B.Cu) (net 8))
 (segment (start 21.7424 90.36304) (end 21.7682 90.33724) (width 0.5) (layer B.Cu) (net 8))
 (segment (start 34.4302 94.88744) (end 34.4302 92.83724) (width 0.5) (layer B.Cu) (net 8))
 (segment (start 32.17788 97.13976) (end 34.4302 94.88744) (width 0.5) (layer B.Cu) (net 8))
 (segment (start 42.95532 97.03816) (end 42.33021 96.41305) (width 0.5) (layer B.Cu) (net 8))
 (segment (start 42.33021 96.41305) (end 42.33021 95.03664) (width 0.5) (layer B.Cu) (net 8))
 (segment (start 42.4302 94.93665) (end 42.4302 92.83724) (width 0.5) (layer B.Cu) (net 8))
 (segment (start 42.33021 95.03664) (end 42.4302 94.93665) (width 0.5) (layer B.Cu) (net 8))
 (segment (start 46.91536 83.93724) (end 44.1302 83.93724) (width 0.5) (layer B.Cu) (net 8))
 (segment (start 47.75708 84.77896) (end 46.91536 83.93724) (width 0.5) (layer B.Cu) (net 8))
 (segment (start 31.695198 86.33724) (end 32.7302 86.33724) (width 0.5) (layer B.Cu) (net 8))
 (segment (start 31.530199 86.172241) (end 31.695198 86.33724) (width 0.5) (layer B.Cu) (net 8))
 (segment (start 31.530199 81.149319) (end 31.530199 86.172241) (width 0.5) (layer B.Cu) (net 8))
 (segment (start 30.31744 79.93656) (end 31.530199 81.149319) (width 0.5) (layer B.Cu) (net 8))
 (segment (start 16.27632 79.15686) (end 16.27632 79.96936) (width 0.25) (layer B.Cu) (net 12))
 (segment (start 19.57852 68.9144) (end 19.57852 69.7894) (width 0.25) (layer B.Cu) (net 12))
 (segment (start 19.57852 69.7894) (end 16.26616 73.10176) (width 0.25) (layer B.Cu) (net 12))
 (segment (start 16.26616 79.1467) (end 16.27632 79.15686) (width 0.25) (layer B.Cu) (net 12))
 (segment (start 16.26616 73.10176) (end 16.26616 79.1467) (width 0.25) (layer B.Cu) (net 12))
 (segment (start 22.90036 73.81744) (end 23.20036 73.81744) (width 0.25) (layer B.Cu) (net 6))
 (segment (start 23.20036 72.50176) (end 23.20036 73.81744) (width 0.25) (layer B.Cu) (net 6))
 (segment (start 23.18512 72.48652) (end 23.20036 72.50176) (width 0.25) (layer B.Cu) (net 6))
 (segment (start 21.56944 72.48652) (end 23.18512 72.48652) (width 0.25) (layer B.Cu) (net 6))
 (segment (start 21.17852 68.9144) (end 21.17852 72.0956) (width 0.25) (layer B.Cu) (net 6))
 (segment (start 21.17852 72.0956) (end 21.56944 72.48652) (width 0.25) (layer B.Cu) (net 6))
 (segment (start 23.20036 75.71744) (end 23.20036 87.05596) (width 0.25) (layer B.Cu) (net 5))
 (segment (start 23.20036 87.05596) (end 24.87168 88.72728) (width 0.25) (layer B.Cu) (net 5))
 (segment (start 20.37852 70.2894) (end 20.36572 70.3022) (width 0.25) (layer B.Cu) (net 4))
 (segment (start 20.37852 68.9144) (end 20.37852 70.2894) (width 0.25) (layer B.Cu) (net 4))
 (segment (start 20.36572 70.3022) (end 20.36572 72.05472) (width 0.25) (layer B.Cu) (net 4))
 (segment (start 19.67484 72.7456) (end 19.67484 73.84796) (width 0.25) (layer B.Cu) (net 4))
 (segment (start 20.36572 72.05472) (end 19.67484 72.7456) (width 0.25) (layer B.Cu) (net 4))
 (segment (start 22.04436 89.53724) (end 32.7302 89.53724) (width 0.25) (layer B.Cu) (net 3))
 (segment (start 19.67484 75.74796) (end 19.67484 87.16772) (width 0.25) (layer B.Cu) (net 3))
 (segment (start 19.67484 87.16772) (end 22.04436 89.53724) (width 0.25) (layer B.Cu) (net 3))
 (segment (start 44.1302 91.17632) (end 44.1302 91.13724) (width 0.25) (layer B.Cu) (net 1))
 (segment (start 47.49264 94.53876) (end 44.1302 91.17632) (width 0.25) (layer B.Cu) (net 1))
 (segment (start 47.79264 94.53876) (end 47.49264 94.53876) (width 0.25) (layer B.Cu) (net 1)))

